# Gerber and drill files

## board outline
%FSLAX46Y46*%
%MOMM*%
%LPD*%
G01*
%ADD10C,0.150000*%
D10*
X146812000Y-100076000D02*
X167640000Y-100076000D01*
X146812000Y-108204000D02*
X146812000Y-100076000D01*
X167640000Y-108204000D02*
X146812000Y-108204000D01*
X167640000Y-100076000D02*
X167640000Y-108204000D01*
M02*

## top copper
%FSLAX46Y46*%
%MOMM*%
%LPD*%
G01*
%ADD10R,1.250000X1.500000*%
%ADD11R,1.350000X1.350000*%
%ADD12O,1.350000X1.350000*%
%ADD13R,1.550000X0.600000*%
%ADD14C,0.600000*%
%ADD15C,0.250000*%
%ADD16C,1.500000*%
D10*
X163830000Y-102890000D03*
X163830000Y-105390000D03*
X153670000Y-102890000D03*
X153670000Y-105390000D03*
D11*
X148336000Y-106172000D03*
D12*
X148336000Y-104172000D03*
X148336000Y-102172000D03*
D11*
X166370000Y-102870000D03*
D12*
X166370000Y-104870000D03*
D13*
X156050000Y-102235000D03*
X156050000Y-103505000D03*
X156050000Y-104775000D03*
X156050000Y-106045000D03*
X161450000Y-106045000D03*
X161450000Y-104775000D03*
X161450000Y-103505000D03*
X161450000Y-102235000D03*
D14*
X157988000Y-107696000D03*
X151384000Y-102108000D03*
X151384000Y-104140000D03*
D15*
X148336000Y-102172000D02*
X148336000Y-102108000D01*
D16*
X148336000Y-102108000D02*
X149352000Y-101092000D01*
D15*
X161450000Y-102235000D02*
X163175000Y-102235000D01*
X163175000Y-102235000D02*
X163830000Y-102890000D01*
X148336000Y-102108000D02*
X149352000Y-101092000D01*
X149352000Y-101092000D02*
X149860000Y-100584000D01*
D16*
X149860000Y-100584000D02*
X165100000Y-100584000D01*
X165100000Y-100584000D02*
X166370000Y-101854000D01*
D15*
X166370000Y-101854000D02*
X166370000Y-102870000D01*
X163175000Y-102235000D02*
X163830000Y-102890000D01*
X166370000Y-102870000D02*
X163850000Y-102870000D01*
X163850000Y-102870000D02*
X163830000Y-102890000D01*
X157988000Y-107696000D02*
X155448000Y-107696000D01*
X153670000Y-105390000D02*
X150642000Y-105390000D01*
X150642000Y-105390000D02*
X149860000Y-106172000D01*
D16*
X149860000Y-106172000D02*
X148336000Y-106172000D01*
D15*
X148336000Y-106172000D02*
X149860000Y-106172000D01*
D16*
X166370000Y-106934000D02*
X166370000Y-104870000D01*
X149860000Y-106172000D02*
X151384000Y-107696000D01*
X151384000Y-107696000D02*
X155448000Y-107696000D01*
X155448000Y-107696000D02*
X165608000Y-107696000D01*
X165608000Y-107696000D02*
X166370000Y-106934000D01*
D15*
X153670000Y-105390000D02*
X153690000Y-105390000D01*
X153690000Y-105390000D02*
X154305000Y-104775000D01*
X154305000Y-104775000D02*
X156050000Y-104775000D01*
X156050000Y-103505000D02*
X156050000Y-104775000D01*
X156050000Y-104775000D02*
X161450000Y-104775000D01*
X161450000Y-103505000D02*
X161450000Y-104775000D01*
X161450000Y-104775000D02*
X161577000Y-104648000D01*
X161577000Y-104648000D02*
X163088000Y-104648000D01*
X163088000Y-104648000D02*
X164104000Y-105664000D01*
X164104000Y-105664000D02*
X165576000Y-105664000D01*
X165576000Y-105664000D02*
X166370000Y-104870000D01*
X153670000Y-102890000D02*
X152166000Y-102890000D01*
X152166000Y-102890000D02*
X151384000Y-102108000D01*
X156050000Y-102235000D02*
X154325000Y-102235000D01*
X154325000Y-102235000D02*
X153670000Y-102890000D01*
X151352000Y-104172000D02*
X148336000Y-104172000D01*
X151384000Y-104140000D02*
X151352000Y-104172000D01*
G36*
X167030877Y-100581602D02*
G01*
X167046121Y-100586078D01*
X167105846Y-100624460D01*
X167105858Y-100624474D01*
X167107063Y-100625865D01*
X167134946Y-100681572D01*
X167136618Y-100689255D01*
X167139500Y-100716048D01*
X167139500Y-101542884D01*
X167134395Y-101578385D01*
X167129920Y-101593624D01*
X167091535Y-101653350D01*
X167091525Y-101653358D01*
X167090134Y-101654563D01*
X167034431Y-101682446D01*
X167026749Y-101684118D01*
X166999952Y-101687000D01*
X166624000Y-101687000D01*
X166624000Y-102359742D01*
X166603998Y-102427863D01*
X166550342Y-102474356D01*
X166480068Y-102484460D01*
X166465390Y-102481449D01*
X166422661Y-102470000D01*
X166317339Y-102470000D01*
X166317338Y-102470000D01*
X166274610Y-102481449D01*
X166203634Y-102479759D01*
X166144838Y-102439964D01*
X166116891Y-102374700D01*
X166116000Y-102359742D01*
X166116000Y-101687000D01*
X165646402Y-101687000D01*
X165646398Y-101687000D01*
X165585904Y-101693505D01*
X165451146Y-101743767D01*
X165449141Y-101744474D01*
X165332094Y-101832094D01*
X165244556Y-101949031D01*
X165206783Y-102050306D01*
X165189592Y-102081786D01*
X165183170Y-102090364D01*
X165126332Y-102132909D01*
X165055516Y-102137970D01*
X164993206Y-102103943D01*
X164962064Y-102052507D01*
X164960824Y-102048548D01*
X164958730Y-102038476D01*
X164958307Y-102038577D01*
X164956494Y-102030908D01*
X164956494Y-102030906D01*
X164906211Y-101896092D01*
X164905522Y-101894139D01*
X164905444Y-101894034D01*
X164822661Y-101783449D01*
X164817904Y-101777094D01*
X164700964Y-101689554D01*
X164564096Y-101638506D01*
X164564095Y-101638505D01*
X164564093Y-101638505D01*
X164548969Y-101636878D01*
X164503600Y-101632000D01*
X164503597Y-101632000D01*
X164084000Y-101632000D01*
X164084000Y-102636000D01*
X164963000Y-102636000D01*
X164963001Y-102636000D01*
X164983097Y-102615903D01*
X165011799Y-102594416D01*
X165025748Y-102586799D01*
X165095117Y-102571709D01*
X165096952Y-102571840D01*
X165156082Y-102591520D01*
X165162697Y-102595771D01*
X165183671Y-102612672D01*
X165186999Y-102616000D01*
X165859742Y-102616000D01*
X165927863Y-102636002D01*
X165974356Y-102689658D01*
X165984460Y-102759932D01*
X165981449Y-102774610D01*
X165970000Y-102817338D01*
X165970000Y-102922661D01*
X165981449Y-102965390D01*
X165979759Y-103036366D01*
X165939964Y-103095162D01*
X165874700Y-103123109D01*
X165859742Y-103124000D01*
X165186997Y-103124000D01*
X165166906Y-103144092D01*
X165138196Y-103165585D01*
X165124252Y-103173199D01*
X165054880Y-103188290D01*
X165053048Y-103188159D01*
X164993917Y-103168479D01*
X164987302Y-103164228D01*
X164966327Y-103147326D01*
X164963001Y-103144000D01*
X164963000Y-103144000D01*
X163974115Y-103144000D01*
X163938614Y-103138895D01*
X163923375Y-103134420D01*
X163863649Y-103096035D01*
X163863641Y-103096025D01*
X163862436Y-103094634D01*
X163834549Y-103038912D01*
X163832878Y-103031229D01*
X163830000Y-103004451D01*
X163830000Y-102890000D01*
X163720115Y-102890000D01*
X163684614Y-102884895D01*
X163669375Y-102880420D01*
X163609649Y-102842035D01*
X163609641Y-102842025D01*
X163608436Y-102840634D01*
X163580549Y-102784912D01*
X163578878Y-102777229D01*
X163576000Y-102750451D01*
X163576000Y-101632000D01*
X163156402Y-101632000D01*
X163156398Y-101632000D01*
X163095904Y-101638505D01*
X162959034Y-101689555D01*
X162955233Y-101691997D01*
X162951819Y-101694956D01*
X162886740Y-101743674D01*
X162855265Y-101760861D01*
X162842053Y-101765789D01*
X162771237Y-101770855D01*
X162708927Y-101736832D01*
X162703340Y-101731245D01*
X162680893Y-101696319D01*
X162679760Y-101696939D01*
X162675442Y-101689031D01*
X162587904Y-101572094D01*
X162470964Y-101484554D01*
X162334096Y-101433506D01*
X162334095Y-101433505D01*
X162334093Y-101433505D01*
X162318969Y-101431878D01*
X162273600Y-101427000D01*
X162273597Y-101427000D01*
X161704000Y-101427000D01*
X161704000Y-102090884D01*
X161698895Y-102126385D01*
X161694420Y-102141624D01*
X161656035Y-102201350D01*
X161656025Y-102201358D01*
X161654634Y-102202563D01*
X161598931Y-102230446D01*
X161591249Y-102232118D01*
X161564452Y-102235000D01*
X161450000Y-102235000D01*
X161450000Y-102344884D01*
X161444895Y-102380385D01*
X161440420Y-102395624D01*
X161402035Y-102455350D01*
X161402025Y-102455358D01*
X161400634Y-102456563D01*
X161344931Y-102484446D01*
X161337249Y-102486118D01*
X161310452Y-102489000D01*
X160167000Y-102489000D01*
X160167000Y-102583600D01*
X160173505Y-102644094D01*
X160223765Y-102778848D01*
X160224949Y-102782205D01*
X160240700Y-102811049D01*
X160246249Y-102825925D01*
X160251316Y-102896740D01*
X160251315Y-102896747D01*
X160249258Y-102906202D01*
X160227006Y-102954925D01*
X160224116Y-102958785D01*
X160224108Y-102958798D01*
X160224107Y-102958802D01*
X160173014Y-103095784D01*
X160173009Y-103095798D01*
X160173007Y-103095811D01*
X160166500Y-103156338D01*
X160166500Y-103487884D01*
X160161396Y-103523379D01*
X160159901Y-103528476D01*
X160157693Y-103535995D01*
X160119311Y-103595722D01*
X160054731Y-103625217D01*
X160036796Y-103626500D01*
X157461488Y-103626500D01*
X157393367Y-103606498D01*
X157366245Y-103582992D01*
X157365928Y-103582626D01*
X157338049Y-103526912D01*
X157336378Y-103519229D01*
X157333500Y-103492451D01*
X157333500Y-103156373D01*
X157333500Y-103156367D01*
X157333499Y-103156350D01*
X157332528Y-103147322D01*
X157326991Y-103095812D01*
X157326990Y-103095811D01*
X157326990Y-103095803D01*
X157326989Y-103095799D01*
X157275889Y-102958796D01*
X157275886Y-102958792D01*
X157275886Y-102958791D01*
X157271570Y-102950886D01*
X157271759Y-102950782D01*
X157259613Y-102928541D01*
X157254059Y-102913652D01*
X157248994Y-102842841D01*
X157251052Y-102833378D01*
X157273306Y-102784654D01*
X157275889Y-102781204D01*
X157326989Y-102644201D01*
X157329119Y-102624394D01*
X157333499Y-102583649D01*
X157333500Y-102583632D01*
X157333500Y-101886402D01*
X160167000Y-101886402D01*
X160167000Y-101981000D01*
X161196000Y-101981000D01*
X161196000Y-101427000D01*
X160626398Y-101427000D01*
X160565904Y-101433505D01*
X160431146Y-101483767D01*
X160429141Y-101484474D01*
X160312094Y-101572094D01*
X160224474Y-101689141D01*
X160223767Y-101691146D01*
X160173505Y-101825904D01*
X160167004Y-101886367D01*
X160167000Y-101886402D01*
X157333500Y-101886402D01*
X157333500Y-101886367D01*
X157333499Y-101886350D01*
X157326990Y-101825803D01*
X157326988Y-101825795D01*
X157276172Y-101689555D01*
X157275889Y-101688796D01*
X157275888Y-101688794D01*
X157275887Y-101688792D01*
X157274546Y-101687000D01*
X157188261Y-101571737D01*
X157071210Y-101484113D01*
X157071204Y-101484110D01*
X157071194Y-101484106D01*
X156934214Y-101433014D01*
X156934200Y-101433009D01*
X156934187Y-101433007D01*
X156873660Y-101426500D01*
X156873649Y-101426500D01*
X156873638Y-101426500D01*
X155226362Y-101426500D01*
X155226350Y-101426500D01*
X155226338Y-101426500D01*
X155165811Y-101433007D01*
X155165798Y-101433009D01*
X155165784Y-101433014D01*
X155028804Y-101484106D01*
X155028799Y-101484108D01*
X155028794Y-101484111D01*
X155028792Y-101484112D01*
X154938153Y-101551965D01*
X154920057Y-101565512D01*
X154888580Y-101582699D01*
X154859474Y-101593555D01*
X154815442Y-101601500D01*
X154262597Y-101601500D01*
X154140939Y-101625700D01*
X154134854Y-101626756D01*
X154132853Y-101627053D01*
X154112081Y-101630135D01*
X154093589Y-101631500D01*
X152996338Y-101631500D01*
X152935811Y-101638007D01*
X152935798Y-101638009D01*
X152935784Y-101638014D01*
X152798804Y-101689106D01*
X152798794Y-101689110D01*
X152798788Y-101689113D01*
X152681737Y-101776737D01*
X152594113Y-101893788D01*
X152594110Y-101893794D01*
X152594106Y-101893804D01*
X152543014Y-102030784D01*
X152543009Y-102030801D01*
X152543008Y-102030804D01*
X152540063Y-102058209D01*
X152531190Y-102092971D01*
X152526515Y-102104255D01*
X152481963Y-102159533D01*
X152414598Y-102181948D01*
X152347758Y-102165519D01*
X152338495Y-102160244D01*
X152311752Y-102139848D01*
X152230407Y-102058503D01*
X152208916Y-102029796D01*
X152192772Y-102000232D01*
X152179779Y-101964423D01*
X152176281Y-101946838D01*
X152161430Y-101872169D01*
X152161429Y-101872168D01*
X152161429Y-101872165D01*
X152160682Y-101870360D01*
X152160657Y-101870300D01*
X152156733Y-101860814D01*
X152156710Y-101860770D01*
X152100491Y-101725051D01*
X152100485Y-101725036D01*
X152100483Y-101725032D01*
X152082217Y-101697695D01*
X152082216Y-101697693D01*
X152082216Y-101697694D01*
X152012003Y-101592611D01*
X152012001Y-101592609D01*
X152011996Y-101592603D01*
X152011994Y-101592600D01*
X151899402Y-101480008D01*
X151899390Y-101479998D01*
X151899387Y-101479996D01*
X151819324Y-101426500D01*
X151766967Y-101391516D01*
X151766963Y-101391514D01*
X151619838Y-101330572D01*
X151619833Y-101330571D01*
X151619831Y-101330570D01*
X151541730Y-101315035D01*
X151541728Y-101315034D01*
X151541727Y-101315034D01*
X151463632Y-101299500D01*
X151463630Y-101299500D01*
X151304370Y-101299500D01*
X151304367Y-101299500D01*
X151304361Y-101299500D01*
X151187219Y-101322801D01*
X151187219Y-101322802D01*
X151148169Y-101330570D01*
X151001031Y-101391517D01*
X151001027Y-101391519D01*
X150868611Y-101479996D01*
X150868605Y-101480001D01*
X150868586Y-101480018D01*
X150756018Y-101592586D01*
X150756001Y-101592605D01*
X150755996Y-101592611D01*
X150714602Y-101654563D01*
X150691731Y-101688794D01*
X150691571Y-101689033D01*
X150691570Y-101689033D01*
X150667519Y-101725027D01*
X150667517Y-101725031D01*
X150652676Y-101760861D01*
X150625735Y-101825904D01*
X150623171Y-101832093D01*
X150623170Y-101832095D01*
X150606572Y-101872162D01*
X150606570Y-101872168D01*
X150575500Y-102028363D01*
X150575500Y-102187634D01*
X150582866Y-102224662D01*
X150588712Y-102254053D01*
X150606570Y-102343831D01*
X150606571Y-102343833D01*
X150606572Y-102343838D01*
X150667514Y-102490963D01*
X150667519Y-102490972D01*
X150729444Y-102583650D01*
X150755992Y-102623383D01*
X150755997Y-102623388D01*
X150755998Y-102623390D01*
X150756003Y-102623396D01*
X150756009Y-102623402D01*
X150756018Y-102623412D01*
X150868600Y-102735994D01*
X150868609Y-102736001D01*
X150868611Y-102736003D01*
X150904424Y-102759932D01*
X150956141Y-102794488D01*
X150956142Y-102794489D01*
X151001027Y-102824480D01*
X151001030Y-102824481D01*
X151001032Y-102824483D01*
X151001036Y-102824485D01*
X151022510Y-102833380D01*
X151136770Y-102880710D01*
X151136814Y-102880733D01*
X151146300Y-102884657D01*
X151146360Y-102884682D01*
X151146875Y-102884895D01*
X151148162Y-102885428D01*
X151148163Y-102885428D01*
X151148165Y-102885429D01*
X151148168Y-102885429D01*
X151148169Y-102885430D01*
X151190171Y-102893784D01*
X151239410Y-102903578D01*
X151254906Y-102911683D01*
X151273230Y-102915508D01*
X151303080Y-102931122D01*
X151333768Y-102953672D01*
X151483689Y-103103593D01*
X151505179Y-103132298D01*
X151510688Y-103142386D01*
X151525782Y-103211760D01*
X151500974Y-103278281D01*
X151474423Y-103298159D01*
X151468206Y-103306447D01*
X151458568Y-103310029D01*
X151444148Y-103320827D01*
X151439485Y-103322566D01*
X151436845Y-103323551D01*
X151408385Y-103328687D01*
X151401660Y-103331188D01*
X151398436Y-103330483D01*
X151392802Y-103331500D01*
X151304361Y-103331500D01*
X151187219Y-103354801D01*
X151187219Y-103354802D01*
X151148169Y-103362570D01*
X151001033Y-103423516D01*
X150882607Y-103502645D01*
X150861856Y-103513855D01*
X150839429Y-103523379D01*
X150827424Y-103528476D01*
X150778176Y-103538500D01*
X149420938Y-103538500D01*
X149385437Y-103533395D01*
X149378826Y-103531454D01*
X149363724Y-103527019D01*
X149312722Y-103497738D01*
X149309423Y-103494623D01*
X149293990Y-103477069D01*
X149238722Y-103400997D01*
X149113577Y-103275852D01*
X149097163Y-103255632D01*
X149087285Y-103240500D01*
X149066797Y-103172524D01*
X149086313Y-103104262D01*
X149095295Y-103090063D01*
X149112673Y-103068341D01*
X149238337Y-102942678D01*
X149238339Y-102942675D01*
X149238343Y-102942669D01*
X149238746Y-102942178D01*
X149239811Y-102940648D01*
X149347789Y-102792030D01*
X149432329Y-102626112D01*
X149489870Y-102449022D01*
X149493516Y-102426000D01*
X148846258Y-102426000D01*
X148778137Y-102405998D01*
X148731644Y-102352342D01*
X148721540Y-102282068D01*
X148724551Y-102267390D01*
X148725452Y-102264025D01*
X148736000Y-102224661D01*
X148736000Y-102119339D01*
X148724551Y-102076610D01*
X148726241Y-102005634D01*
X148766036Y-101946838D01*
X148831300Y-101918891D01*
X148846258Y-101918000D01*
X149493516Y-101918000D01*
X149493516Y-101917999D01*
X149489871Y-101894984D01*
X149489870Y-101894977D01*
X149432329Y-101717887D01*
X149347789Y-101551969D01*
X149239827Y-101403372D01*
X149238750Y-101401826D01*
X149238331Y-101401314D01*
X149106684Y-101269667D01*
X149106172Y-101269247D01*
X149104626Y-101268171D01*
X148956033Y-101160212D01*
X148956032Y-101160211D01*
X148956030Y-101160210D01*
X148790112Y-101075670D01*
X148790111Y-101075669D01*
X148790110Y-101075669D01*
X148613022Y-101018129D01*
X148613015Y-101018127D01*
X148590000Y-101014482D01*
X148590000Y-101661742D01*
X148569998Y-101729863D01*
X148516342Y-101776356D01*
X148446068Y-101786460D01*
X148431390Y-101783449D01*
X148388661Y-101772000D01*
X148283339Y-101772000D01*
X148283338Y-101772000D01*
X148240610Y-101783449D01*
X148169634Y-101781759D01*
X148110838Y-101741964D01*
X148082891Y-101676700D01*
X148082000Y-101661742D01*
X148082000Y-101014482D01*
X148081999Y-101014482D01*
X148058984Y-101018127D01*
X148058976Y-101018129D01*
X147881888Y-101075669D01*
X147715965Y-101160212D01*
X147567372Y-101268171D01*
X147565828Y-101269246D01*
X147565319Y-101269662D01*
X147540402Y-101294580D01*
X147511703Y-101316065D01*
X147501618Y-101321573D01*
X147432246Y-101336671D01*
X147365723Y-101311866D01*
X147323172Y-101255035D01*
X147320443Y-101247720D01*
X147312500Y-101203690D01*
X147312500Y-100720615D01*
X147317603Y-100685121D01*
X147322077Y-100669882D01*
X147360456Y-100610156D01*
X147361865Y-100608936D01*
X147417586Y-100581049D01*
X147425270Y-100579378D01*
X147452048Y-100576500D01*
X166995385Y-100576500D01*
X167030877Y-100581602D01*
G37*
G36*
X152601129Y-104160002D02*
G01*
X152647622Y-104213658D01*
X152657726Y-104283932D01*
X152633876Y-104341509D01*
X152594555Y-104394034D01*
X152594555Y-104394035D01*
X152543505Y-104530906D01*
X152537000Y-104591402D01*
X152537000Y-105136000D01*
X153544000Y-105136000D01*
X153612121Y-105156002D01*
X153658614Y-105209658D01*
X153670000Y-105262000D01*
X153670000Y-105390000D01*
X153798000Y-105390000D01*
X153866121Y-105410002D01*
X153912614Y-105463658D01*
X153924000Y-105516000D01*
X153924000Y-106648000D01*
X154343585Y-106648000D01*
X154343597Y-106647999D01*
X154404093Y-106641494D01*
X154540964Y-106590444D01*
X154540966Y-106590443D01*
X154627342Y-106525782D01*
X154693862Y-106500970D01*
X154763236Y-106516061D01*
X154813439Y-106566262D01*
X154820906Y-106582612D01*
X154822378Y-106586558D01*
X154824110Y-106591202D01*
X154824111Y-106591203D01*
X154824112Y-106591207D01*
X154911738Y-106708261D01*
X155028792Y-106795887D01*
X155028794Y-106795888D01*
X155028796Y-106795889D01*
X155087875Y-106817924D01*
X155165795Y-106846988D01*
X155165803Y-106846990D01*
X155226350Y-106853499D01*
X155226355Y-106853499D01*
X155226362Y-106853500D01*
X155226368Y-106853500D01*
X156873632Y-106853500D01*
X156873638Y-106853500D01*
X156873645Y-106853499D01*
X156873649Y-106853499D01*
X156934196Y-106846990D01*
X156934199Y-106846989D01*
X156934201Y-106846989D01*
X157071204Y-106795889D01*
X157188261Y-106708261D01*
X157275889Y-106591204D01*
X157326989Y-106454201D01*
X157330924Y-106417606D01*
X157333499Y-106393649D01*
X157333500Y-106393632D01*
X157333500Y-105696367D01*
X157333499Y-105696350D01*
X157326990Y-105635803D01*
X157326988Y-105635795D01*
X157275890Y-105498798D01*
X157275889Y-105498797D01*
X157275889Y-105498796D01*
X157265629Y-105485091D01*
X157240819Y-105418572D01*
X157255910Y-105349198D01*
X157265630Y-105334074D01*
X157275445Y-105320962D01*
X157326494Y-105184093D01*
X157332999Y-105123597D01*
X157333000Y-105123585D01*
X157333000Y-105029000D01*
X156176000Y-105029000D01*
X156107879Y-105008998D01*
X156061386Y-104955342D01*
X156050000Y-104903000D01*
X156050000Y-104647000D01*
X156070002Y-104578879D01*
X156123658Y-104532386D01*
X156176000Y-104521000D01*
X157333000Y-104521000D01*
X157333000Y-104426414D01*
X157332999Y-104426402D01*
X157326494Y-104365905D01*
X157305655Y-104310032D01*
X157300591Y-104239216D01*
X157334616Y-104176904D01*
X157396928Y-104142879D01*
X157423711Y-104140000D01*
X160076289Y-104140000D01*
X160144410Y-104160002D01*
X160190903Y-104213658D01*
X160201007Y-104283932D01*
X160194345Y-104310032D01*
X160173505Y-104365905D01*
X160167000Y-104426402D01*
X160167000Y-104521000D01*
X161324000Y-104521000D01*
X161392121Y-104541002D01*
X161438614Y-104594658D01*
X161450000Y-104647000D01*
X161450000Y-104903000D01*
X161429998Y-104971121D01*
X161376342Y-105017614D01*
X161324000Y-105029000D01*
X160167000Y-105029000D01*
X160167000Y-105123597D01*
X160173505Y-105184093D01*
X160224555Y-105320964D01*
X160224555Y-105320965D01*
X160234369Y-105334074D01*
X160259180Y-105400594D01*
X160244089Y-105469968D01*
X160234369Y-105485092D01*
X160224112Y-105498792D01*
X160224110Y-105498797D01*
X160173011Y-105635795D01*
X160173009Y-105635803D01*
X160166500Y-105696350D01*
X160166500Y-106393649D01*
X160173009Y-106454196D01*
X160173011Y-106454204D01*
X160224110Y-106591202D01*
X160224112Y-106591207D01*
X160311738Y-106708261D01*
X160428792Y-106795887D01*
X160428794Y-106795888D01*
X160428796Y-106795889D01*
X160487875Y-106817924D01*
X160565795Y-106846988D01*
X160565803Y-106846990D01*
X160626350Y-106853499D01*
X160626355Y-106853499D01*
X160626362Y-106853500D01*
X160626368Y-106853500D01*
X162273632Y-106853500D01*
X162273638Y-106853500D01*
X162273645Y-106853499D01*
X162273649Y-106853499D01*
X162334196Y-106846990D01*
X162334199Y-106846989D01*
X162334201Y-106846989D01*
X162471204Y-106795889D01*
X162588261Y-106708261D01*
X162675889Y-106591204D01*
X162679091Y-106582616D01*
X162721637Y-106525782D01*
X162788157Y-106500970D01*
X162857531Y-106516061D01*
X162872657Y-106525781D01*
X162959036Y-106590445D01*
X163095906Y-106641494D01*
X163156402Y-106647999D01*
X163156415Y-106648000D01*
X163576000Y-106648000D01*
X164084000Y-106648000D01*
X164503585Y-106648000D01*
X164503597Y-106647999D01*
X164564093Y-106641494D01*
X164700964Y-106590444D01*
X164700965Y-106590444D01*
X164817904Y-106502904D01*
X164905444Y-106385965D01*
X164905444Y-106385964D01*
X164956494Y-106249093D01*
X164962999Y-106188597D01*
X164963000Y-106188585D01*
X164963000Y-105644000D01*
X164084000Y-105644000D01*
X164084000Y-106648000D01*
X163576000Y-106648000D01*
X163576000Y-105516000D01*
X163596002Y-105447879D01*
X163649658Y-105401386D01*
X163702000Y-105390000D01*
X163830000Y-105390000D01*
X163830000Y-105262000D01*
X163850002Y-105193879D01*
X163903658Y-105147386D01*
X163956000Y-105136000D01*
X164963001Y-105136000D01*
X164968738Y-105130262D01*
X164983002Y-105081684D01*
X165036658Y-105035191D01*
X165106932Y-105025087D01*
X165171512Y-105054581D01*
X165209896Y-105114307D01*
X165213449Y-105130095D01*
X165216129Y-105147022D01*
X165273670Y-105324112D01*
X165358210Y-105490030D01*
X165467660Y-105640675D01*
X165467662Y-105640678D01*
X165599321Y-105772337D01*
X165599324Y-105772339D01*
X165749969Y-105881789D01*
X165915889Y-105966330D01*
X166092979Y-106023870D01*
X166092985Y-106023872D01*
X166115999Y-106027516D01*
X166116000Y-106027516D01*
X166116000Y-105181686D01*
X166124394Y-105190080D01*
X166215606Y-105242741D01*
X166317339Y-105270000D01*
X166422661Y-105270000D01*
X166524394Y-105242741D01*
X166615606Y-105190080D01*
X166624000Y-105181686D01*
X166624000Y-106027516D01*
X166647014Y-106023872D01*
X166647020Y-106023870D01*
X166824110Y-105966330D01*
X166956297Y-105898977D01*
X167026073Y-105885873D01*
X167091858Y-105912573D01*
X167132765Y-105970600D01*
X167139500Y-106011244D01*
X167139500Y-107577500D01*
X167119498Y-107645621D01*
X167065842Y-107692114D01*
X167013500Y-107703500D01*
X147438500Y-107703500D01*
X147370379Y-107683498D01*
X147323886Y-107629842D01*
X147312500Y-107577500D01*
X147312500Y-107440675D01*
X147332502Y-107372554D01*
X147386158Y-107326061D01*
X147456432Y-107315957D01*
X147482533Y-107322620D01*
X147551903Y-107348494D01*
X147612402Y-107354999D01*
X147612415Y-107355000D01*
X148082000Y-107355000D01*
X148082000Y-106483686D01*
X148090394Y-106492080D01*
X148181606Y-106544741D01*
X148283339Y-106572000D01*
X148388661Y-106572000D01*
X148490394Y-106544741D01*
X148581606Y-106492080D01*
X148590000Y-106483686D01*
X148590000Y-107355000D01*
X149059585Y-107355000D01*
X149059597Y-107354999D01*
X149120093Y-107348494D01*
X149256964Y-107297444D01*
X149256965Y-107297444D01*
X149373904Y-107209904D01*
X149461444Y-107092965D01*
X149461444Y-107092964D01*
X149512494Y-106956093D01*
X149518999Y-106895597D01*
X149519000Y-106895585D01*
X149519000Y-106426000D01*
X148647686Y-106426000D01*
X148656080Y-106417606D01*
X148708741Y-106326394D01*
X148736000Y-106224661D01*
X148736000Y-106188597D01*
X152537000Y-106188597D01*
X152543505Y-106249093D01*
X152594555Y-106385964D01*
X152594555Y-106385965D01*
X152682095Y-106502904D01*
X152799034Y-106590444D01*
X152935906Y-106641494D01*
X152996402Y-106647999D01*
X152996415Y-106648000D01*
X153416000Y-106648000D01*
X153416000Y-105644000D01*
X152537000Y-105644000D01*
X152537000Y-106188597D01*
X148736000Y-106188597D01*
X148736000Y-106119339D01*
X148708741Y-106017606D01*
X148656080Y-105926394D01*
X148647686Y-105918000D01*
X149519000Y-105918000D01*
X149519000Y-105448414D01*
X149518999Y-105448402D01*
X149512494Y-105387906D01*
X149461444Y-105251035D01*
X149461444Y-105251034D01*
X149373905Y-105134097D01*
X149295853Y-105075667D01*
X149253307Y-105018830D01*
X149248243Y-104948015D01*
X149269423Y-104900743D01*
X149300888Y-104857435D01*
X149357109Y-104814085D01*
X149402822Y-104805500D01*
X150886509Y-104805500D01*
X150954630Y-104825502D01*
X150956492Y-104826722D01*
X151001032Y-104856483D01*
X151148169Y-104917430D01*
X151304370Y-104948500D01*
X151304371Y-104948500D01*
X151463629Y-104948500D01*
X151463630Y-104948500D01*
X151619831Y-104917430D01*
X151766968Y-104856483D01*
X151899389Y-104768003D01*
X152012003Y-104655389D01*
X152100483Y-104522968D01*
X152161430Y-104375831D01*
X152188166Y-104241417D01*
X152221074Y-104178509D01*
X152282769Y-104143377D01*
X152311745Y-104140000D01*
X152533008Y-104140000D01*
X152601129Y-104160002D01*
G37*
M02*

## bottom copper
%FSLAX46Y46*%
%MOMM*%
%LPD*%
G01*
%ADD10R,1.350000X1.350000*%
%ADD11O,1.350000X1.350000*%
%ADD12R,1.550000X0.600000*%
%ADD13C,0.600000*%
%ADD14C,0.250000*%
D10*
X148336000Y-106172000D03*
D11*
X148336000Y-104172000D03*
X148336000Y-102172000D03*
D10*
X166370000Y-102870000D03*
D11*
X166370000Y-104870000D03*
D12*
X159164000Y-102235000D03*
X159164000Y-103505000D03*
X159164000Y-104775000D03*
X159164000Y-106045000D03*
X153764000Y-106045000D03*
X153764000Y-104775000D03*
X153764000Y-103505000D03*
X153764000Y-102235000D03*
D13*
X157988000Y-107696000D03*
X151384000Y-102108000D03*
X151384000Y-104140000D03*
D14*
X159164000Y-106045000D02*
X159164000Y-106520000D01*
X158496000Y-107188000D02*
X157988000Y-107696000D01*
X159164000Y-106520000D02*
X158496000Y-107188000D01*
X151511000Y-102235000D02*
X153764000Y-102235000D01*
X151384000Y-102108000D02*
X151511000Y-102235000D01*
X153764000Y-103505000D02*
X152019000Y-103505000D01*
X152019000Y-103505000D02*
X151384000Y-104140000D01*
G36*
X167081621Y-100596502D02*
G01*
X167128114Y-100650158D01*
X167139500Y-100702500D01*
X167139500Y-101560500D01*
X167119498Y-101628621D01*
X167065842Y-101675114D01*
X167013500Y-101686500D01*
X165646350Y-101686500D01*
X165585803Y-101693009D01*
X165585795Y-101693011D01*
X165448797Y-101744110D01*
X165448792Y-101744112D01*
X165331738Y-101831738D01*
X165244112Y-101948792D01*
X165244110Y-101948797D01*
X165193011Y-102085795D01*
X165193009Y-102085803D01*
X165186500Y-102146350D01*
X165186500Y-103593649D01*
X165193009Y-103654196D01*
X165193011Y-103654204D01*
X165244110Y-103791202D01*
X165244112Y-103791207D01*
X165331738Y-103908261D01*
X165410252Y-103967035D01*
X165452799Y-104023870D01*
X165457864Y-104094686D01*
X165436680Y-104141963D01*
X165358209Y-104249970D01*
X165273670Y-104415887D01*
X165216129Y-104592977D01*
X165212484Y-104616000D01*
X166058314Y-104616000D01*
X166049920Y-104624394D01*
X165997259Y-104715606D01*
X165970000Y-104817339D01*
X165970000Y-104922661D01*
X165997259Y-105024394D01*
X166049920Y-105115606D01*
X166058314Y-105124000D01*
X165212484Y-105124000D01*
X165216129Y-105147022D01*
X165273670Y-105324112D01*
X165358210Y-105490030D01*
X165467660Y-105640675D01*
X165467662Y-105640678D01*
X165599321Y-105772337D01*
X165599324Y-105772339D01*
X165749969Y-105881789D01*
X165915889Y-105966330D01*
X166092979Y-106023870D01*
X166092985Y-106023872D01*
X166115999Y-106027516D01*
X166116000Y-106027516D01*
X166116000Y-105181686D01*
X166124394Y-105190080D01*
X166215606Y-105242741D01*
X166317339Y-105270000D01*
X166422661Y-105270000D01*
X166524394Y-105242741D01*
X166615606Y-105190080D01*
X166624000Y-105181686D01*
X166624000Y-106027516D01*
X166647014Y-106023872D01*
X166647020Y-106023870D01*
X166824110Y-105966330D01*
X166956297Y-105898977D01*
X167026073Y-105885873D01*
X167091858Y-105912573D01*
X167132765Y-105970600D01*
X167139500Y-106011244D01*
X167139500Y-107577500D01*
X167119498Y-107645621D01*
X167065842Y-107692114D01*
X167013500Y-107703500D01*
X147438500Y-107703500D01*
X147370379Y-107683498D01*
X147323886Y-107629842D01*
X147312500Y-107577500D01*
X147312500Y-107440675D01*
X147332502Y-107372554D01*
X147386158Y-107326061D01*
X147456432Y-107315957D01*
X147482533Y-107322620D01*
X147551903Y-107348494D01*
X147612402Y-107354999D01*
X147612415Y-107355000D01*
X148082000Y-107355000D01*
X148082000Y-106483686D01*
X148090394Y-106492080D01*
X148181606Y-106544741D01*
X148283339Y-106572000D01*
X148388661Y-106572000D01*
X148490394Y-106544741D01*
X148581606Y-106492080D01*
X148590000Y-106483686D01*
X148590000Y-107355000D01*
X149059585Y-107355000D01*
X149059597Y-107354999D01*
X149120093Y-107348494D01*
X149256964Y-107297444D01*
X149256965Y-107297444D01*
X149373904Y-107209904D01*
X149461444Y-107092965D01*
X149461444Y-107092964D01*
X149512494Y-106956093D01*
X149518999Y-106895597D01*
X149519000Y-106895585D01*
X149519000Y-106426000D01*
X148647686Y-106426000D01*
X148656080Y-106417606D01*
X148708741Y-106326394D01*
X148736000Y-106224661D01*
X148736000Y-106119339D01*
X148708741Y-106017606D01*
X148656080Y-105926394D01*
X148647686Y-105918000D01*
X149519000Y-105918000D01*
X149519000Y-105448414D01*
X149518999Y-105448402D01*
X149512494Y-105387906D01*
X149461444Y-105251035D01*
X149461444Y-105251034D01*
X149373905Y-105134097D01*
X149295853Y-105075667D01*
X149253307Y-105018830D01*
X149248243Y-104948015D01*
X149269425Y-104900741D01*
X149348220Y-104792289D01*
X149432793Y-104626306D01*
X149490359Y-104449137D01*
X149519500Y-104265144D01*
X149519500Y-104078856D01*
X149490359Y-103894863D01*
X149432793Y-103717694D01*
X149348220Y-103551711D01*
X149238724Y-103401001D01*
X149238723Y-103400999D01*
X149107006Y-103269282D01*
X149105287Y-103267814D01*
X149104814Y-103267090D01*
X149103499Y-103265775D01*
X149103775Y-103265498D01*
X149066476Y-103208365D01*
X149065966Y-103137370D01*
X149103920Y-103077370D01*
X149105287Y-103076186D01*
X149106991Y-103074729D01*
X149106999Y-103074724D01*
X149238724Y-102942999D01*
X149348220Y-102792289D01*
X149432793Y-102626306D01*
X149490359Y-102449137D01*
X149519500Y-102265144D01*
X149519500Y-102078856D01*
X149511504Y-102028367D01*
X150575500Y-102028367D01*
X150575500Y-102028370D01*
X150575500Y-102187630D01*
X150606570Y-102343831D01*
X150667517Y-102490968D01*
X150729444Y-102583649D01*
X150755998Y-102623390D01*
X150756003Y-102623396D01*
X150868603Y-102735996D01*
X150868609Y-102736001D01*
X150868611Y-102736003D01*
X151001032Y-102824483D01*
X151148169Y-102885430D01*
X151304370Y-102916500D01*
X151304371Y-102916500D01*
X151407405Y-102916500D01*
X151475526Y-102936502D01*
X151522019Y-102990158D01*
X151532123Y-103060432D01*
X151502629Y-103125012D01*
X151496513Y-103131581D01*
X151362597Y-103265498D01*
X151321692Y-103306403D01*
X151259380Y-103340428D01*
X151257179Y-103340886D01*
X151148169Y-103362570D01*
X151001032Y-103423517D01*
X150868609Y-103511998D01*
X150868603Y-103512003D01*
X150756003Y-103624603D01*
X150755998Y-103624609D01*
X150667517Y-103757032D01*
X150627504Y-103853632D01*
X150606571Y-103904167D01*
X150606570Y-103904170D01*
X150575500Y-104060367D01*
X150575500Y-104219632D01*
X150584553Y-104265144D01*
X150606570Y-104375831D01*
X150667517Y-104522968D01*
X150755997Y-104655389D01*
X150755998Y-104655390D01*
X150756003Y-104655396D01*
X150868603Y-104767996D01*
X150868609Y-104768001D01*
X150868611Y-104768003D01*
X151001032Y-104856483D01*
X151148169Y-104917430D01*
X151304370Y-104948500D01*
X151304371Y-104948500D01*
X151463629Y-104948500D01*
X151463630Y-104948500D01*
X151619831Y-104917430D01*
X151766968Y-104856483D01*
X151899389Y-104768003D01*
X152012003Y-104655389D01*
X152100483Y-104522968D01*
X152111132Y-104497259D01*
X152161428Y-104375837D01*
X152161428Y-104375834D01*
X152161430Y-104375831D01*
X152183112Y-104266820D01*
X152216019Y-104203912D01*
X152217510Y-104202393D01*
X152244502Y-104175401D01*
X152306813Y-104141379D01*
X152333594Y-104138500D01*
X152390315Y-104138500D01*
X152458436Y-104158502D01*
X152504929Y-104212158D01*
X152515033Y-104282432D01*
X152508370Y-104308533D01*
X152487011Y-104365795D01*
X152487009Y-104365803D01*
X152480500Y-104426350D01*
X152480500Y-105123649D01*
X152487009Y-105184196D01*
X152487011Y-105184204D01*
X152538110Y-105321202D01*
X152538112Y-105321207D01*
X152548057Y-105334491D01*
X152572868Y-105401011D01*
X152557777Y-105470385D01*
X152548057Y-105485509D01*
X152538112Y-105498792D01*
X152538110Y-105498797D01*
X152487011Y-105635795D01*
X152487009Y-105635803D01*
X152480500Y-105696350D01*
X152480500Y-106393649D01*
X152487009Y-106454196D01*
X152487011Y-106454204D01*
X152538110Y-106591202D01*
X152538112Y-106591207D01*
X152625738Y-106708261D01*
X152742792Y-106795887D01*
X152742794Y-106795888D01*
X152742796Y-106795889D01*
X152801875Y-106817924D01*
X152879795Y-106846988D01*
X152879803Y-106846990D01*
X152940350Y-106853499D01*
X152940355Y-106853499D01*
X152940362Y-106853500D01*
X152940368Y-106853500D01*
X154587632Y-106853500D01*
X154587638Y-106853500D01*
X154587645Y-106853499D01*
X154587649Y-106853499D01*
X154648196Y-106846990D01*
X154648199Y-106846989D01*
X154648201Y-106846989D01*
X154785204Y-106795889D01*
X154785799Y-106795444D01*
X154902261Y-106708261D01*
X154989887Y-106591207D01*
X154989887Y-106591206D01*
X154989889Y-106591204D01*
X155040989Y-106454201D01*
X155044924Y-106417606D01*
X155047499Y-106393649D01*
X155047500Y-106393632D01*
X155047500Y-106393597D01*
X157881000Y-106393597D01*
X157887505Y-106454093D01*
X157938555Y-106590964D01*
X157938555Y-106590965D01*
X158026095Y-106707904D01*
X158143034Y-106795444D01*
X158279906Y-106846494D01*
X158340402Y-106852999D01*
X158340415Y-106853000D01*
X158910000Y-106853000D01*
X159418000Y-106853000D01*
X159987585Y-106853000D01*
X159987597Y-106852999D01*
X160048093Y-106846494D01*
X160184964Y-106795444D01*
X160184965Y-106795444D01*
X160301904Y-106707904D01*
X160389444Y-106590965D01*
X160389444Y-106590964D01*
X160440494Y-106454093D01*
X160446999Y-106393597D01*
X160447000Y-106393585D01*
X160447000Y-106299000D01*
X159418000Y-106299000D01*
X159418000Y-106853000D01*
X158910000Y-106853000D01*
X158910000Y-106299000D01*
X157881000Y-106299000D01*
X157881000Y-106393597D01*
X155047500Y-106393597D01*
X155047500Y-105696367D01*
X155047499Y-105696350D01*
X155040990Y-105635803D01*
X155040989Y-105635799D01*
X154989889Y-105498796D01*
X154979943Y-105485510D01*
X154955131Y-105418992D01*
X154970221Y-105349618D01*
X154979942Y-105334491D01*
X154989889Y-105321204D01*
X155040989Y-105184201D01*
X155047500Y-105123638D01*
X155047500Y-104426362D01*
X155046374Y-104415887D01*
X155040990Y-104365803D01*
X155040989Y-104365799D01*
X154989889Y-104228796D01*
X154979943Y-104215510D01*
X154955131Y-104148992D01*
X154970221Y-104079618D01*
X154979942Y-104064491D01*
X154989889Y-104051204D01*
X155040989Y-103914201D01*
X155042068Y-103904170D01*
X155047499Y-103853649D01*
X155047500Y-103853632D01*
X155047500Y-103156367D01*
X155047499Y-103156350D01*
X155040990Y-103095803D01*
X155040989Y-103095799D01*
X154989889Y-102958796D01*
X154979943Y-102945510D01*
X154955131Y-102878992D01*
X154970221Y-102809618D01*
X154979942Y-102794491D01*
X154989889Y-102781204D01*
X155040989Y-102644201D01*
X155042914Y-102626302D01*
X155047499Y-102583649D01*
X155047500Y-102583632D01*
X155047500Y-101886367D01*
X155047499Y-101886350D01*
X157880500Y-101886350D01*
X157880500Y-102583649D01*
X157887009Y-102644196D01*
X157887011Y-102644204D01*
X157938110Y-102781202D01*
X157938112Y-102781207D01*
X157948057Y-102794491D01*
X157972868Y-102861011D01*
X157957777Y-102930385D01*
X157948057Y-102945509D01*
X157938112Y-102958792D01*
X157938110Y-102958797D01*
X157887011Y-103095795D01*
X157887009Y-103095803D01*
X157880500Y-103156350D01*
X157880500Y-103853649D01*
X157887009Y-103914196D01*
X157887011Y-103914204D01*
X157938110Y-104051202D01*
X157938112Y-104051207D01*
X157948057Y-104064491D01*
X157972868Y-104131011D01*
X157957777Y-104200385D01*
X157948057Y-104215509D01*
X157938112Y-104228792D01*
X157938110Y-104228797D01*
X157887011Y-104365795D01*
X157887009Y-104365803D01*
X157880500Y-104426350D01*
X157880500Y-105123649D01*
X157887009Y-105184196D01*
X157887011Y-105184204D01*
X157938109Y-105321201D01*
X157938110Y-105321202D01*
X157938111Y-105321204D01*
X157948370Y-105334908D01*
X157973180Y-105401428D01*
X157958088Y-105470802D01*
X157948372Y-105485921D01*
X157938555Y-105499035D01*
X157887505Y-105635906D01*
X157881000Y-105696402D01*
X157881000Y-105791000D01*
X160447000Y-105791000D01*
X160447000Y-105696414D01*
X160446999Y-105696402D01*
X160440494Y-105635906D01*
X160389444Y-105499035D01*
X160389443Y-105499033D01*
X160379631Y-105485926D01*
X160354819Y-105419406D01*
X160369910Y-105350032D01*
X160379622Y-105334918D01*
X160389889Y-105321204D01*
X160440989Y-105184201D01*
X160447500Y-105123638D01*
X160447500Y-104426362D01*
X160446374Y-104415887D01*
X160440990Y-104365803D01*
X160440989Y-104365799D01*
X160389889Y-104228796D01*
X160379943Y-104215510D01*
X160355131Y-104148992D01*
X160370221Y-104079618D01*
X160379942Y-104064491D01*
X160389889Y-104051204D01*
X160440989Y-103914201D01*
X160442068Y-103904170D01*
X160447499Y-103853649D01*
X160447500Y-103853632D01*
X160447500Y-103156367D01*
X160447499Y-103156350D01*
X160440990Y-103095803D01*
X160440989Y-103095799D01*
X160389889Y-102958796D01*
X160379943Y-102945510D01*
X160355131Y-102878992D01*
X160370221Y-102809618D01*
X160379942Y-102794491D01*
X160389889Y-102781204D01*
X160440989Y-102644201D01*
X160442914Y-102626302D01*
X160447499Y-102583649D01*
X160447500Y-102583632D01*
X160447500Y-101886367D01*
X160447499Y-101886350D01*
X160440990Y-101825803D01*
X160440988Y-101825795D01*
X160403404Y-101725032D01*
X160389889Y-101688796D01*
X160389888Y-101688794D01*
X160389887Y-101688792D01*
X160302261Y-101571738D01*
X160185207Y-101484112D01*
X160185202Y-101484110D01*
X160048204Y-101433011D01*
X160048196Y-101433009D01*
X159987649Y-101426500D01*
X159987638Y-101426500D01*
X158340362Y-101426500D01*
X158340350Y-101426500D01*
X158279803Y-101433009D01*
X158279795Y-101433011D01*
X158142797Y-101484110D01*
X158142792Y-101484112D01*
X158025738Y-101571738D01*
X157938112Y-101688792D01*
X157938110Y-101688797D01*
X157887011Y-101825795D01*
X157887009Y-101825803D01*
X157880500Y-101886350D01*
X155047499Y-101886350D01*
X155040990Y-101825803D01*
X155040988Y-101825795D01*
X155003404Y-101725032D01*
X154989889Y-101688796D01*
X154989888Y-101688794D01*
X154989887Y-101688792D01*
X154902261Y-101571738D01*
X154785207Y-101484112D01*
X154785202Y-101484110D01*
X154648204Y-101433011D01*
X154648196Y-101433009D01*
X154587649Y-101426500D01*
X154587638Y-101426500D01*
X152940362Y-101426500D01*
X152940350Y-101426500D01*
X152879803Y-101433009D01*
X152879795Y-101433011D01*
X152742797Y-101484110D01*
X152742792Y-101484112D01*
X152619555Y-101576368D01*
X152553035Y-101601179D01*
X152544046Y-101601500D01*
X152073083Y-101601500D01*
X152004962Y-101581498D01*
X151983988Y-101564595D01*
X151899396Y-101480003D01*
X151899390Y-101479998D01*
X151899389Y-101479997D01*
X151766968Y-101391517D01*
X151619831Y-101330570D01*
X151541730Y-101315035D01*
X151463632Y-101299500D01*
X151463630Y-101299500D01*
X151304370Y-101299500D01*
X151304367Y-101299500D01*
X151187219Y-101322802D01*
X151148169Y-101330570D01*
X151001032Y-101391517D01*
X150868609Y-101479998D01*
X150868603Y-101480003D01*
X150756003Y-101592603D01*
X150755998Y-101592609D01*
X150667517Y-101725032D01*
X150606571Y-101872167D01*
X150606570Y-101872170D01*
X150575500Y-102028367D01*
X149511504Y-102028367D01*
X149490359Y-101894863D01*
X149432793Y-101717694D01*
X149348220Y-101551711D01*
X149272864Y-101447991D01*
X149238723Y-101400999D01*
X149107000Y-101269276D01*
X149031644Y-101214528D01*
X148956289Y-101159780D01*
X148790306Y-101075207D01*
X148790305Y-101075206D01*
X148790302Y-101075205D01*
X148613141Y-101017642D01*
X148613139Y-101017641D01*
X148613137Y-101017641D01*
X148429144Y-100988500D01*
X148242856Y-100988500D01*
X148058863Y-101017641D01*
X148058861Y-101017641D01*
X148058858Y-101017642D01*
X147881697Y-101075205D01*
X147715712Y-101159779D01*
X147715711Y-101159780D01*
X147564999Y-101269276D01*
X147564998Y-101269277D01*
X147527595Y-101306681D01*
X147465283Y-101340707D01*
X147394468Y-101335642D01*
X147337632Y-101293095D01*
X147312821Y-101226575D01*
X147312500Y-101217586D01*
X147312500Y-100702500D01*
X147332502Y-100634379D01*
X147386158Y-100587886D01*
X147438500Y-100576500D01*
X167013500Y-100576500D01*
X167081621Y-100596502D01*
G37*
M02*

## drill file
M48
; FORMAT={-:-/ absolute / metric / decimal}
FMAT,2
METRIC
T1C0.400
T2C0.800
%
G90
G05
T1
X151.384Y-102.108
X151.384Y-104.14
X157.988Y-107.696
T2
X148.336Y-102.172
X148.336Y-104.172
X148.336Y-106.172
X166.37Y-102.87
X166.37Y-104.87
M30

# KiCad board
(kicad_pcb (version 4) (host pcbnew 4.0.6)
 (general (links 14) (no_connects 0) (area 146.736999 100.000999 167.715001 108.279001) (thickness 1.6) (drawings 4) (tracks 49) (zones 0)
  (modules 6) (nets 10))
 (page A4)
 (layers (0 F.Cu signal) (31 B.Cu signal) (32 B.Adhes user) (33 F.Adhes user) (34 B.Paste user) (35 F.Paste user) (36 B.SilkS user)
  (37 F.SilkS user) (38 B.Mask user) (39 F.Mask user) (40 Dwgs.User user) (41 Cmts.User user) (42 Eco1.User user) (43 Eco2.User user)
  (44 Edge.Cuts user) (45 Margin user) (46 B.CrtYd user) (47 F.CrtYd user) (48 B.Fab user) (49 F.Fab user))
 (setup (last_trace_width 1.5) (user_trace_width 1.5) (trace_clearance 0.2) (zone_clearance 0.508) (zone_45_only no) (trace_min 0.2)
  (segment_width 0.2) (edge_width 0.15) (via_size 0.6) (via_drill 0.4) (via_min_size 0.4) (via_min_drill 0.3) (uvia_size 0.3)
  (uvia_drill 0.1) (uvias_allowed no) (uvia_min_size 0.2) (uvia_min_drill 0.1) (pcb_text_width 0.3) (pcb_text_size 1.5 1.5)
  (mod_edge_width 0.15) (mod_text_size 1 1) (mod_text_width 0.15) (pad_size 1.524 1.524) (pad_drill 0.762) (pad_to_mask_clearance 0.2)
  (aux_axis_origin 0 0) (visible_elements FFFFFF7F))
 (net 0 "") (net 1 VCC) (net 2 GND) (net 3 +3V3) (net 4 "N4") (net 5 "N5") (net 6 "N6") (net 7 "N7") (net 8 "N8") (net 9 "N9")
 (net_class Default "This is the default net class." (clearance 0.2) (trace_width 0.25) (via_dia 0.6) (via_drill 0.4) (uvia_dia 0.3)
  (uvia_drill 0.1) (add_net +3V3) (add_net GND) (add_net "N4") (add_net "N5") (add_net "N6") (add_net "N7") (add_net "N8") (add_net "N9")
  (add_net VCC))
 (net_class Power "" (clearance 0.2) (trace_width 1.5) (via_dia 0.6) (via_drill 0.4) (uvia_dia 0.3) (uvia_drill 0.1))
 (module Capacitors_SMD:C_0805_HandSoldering (layer F.Cu) (at 163.83 104.14 270)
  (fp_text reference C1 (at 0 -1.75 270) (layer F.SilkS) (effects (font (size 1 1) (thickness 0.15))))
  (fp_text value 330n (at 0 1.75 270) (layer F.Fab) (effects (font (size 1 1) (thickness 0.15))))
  (pad 1 smd rect (at -1.25 0 270) (size 1.5 1.25) (layers F.Cu F.Paste F.Mask) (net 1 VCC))
  (pad 2 smd rect (at 1.25 0 270) (size 1.5 1.25) (layers F.Cu F.Paste F.Mask) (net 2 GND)))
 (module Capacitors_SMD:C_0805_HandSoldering (layer F.Cu) (at 153.67 104.14 270)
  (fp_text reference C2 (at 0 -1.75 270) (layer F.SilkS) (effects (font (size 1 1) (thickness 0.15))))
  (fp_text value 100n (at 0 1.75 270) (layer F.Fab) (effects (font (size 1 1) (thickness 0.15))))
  (pad 1 smd rect (at -1.25 0 270) (size 1.5 1.25) (layers F.Cu F.Paste F.Mask) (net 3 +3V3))
  (pad 2 smd rect (at 1.25 0 270) (size 1.5 1.25) (layers F.Cu F.Paste F.Mask) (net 2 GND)))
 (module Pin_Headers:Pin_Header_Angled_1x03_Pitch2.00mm (layer F.Cu) (at 148.336 106.172 180)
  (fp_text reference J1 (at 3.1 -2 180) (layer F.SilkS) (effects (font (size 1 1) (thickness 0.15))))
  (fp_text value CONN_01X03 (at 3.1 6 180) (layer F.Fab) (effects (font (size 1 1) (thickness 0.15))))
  (pad 1 thru_hole rect (at 0 0 180) (size 1.35 1.35) (drill 0.8) (layers *.Cu *.Mask) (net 2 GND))
  (pad 2 thru_hole oval (at 0 2 180) (size 1.35 1.35) (drill 0.8) (layers *.Cu *.Mask) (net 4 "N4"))
  (pad 3 thru_hole oval (at 0 4 180) (size 1.35 1.35) (drill 0.8) (layers *.Cu *.Mask) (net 1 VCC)))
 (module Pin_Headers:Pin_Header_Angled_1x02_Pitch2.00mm (layer F.Cu) (at 166.37 102.87)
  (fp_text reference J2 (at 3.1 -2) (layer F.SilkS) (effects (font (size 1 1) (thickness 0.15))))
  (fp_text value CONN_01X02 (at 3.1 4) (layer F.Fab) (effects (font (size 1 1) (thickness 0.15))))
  (pad 1 thru_hole rect (at 0 0) (size 1.35 1.35) (drill 0.8) (layers *.Cu *.Mask) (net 1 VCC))
  (pad 2 thru_hole oval (at 0 2) (size 1.35 1.35) (drill 0.8) (layers *.Cu *.Mask) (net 2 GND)))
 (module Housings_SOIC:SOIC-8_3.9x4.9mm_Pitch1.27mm (layer B.Cu) (at 156.464 104.14 180)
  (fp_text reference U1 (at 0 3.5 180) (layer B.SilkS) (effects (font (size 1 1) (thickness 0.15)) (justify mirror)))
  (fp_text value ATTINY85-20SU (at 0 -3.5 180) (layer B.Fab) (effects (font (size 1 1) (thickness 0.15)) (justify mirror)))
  (pad 1 smd rect (at -2.7 1.905 180) (size 1.55 0.6) (layers B.Cu B.Paste B.Mask) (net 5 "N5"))
  (pad 2 smd rect (at -2.7 0.635 180) (size 1.55 0.6) (layers B.Cu B.Paste B.Mask) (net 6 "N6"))
  (pad 3 smd rect (at -2.7 -0.635 180) (size 1.55 0.6) (layers B.Cu B.Paste B.Mask) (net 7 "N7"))
  (pad 4 smd rect (at -2.7 -1.905 180) (size 1.55 0.6) (layers B.Cu B.Paste B.Mask) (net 2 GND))
  (pad 5 smd rect (at 2.7 -1.905 180) (size 1.55 0.6) (layers B.Cu B.Paste B.Mask) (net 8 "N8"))
  (pad 6 smd rect (at 2.7 -0.635 180) (size 1.55 0.6) (layers B.Cu B.Paste B.Mask) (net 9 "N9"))
  (pad 7 smd rect (at 2.7 0.635 180) (size 1.55 0.6) (layers B.Cu B.Paste B.Mask) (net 4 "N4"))
  (pad 8 smd rect (at 2.7 1.905 180) (size 1.55 0.6) (layers B.Cu B.Paste B.Mask) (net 3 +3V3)))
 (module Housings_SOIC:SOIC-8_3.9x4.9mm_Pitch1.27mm (layer F.Cu) (at 158.75 104.14)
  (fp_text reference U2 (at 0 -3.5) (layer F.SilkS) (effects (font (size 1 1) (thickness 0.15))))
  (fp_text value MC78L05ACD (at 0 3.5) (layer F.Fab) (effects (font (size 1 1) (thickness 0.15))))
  (pad 1 smd rect (at -2.7 -1.905) (size 1.55 0.6) (layers F.Cu F.Paste F.Mask) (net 3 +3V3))
  (pad 2 smd rect (at -2.7 -0.635) (size 1.55 0.6) (layers F.Cu F.Paste F.Mask) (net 2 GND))
  (pad 3 smd rect (at -2.7 0.635) (size 1.55 0.6) (layers F.Cu F.Paste F.Mask) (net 2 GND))
  (pad 4 smd rect (at -2.7 1.905) (size 1.55 0.6) (layers F.Cu F.Paste F.Mask))
  (pad 5 smd rect (at 2.7 1.905) (size 1.55 0.6) (layers F.Cu F.Paste F.Mask))
  (pad 6 smd rect (at 2.7 0.635) (size 1.55 0.6) (layers F.Cu F.Paste F.Mask) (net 2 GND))
  (pad 7 smd rect (at 2.7 -0.635) (size 1.55 0.6) (layers F.Cu F.Paste F.Mask) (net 2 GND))
  (pad 8 smd rect (at 2.7 -1.905) (size 1.55 0.6) (layers F.Cu F.Paste F.Mask) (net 1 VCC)))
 (gr_line (start 146.812 100.076) (end 167.64 100.076) (angle 90) (layer Edge.Cuts) (width 0.15))
 (gr_line (start 146.812 108.204) (end 146.812 100.076) (angle 90) (layer Edge.Cuts) (width 0.15))
 (gr_line (start 167.64 108.204) (end 146.812 108.204) (angle 90) (layer Edge.Cuts) (width 0.15))
 (gr_line (start 167.64 100.076) (end 167.64 108.204) (angle 90) (layer Edge.Cuts) (width 0.15))
 (segment (start 148.336 102.172) (end 148.336 102.108) (width 0.25) (layer F.Cu) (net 1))
 (segment (start 148.336 102.108) (end 149.352 101.092) (width 1.5) (layer F.Cu) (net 1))
 (segment (start 161.45 102.235) (end 163.175 102.235) (width 0.25) (layer F.Cu) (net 1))
 (segment (start 163.175 102.235) (end 163.83 102.89) (width 0.25) (layer F.Cu) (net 1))
 (segment (start 148.336 102.108) (end 149.352 101.092) (width 0.25) (layer F.Cu) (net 1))
 (segment (start 149.352 101.092) (end 149.86 100.584) (width 0.25) (layer F.Cu) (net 1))
 (segment (start 149.86 100.584) (end 165.1 100.584) (width 1.5) (layer F.Cu) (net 1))
 (segment (start 165.1 100.584) (end 166.37 101.854) (width 1.5) (layer F.Cu) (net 1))
 (segment (start 166.37 101.854) (end 166.37 102.87) (width 0.25) (layer F.Cu) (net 1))
 (segment (start 163.175 102.235) (end 163.83 102.89) (width 0.25) (layer F.Cu) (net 1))
 (segment (start 166.37 102.87) (end 163.85 102.87) (width 0.25) (layer F.Cu) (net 1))
 (segment (start 163.85 102.87) (end 163.83 102.89) (width 0.25) (layer F.Cu) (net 1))
 (segment (start 159.164 106.045) (end 159.164 106.52) (width 0.25) (layer B.Cu) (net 2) (status 400000))
 (segment (start 157.988 107.696) (end 155.448 107.696) (width 0.25) (layer F.Cu) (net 2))
 (via (at 157.988 107.696) (size 0.6) (drill 0.4) (layers F.Cu B.Cu) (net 2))
 (segment (start 158.496 107.188) (end 157.988 107.696) (width 0.25) (layer B.Cu) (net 2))
 (segment (start 159.164 106.52) (end 158.496 107.188) (width 0.25) (layer B.Cu) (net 2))
 (segment (start 153.67 105.39) (end 150.642 105.39) (width 0.25) (layer F.Cu) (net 2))
 (segment (start 150.642 105.39) (end 149.86 106.172) (width 0.25) (layer F.Cu) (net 2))
 (segment (start 149.86 106.172) (end 148.336 106.172) (width 1.5) (layer F.Cu) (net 2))
 (segment (start 148.336 106.172) (end 149.86 106.172) (width 0.25) (layer F.Cu) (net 2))
 (segment (start 166.37 106.934) (end 166.37 104.87) (width 1.5) (layer F.Cu) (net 2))
 (segment (start 149.86 106.172) (end 151.384 107.696) (width 1.5) (layer F.Cu) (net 2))
 (segment (start 151.384 107.696) (end 155.448 107.696) (width 1.5) (layer F.Cu) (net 2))
 (segment (start 155.448 107.696) (end 165.608 107.696) (width 1.5) (layer F.Cu) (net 2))
 (segment (start 165.608 107.696) (end 166.37 106.934) (width 1.5) (layer F.Cu) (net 2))
 (segment (start 153.67 105.39) (end 153.69 105.39) (width 0.25) (layer F.Cu) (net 2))
 (segment (start 153.69 105.39) (end 154.305 104.775) (width 0.25) (layer F.Cu) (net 2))
 (segment (start 154.305 104.775) (end 156.05 104.775) (width 0.25) (layer F.Cu) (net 2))
 (segment (start 156.05 103.505) (end 156.05 104.775) (width 0.25) (layer F.Cu) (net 2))
 (segment (start 156.05 104.775) (end 161.45 104.775) (width 0.25) (layer F.Cu) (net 2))
 (segment (start 161.45 103.505) (end 161.45 104.775) (width 0.25) (layer F.Cu) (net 2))
 (segment (start 161.45 104.775) (end 161.577 104.648) (width 0.25) (layer F.Cu) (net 2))
 (segment (start 161.577 104.648) (end 163.088 104.648) (width 0.25) (layer F.Cu) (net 2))
 (segment (start 163.088 104.648) (end 164.104 105.664) (width 0.25) (layer F.Cu) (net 2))
 (segment (start 164.104 105.664) (end 165.576 105.664) (width 0.25) (layer F.Cu) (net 2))
 (segment (start 165.576 105.664) (end 166.37 104.87) (width 0.25) (layer F.Cu) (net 2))
 (segment (start 153.67 102.89) (end 152.166 102.89) (width 0.25) (layer F.Cu) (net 3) (status 400000))
 (segment (start 151.511 102.235) (end 153.764 102.235) (width 0.25) (layer B.Cu) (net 3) (status 800000))
 (segment (start 151.384 102.108) (end 151.511 102.235) (width 0.25) (layer B.Cu) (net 3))
 (via (at 151.384 102.108) (size 0.6) (drill 0.4) (layers F.Cu B.Cu) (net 3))
 (segment (start 152.166 102.89) (end 151.384 102.108) (width 0.25) (layer F.Cu) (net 3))
 (segment (start 156.05 102.235) (end 154.325 102.235) (width 0.25) (layer F.Cu) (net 3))
 (segment (start 154.325 102.235) (end 153.67 102.89) (width 0.25) (layer F.Cu) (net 3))
 (segment (start 153.764 103.505) (end 152.019 103.505) (width 0.25) (layer B.Cu) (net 4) (status 400000))
 (segment (start 151.352 104.172) (end 148.336 104.172) (width 0.25) (layer F.Cu) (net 4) (status 800000))
 (segment (start 151.384 104.14) (end 151.352 104.172) (width 0.25) (layer F.Cu) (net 4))
 (via (at 151.384 104.14) (size 0.6) (drill 0.4) (layers F.Cu B.Cu) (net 4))
 (segment (start 152.019 103.505) (end 151.384 104.14) (width 0.25) (layer B.Cu) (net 4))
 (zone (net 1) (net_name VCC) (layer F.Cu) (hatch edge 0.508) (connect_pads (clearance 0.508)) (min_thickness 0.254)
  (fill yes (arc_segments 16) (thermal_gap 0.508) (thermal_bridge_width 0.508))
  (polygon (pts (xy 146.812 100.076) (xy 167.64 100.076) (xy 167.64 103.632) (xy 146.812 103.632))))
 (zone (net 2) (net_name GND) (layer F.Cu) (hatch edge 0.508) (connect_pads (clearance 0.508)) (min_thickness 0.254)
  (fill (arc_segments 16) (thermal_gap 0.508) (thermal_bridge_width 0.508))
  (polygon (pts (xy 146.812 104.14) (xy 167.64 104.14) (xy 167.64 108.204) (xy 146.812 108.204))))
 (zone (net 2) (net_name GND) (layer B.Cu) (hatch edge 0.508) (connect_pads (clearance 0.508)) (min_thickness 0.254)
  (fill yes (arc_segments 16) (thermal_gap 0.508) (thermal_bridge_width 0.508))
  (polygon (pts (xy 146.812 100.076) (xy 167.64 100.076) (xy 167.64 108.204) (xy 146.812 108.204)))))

